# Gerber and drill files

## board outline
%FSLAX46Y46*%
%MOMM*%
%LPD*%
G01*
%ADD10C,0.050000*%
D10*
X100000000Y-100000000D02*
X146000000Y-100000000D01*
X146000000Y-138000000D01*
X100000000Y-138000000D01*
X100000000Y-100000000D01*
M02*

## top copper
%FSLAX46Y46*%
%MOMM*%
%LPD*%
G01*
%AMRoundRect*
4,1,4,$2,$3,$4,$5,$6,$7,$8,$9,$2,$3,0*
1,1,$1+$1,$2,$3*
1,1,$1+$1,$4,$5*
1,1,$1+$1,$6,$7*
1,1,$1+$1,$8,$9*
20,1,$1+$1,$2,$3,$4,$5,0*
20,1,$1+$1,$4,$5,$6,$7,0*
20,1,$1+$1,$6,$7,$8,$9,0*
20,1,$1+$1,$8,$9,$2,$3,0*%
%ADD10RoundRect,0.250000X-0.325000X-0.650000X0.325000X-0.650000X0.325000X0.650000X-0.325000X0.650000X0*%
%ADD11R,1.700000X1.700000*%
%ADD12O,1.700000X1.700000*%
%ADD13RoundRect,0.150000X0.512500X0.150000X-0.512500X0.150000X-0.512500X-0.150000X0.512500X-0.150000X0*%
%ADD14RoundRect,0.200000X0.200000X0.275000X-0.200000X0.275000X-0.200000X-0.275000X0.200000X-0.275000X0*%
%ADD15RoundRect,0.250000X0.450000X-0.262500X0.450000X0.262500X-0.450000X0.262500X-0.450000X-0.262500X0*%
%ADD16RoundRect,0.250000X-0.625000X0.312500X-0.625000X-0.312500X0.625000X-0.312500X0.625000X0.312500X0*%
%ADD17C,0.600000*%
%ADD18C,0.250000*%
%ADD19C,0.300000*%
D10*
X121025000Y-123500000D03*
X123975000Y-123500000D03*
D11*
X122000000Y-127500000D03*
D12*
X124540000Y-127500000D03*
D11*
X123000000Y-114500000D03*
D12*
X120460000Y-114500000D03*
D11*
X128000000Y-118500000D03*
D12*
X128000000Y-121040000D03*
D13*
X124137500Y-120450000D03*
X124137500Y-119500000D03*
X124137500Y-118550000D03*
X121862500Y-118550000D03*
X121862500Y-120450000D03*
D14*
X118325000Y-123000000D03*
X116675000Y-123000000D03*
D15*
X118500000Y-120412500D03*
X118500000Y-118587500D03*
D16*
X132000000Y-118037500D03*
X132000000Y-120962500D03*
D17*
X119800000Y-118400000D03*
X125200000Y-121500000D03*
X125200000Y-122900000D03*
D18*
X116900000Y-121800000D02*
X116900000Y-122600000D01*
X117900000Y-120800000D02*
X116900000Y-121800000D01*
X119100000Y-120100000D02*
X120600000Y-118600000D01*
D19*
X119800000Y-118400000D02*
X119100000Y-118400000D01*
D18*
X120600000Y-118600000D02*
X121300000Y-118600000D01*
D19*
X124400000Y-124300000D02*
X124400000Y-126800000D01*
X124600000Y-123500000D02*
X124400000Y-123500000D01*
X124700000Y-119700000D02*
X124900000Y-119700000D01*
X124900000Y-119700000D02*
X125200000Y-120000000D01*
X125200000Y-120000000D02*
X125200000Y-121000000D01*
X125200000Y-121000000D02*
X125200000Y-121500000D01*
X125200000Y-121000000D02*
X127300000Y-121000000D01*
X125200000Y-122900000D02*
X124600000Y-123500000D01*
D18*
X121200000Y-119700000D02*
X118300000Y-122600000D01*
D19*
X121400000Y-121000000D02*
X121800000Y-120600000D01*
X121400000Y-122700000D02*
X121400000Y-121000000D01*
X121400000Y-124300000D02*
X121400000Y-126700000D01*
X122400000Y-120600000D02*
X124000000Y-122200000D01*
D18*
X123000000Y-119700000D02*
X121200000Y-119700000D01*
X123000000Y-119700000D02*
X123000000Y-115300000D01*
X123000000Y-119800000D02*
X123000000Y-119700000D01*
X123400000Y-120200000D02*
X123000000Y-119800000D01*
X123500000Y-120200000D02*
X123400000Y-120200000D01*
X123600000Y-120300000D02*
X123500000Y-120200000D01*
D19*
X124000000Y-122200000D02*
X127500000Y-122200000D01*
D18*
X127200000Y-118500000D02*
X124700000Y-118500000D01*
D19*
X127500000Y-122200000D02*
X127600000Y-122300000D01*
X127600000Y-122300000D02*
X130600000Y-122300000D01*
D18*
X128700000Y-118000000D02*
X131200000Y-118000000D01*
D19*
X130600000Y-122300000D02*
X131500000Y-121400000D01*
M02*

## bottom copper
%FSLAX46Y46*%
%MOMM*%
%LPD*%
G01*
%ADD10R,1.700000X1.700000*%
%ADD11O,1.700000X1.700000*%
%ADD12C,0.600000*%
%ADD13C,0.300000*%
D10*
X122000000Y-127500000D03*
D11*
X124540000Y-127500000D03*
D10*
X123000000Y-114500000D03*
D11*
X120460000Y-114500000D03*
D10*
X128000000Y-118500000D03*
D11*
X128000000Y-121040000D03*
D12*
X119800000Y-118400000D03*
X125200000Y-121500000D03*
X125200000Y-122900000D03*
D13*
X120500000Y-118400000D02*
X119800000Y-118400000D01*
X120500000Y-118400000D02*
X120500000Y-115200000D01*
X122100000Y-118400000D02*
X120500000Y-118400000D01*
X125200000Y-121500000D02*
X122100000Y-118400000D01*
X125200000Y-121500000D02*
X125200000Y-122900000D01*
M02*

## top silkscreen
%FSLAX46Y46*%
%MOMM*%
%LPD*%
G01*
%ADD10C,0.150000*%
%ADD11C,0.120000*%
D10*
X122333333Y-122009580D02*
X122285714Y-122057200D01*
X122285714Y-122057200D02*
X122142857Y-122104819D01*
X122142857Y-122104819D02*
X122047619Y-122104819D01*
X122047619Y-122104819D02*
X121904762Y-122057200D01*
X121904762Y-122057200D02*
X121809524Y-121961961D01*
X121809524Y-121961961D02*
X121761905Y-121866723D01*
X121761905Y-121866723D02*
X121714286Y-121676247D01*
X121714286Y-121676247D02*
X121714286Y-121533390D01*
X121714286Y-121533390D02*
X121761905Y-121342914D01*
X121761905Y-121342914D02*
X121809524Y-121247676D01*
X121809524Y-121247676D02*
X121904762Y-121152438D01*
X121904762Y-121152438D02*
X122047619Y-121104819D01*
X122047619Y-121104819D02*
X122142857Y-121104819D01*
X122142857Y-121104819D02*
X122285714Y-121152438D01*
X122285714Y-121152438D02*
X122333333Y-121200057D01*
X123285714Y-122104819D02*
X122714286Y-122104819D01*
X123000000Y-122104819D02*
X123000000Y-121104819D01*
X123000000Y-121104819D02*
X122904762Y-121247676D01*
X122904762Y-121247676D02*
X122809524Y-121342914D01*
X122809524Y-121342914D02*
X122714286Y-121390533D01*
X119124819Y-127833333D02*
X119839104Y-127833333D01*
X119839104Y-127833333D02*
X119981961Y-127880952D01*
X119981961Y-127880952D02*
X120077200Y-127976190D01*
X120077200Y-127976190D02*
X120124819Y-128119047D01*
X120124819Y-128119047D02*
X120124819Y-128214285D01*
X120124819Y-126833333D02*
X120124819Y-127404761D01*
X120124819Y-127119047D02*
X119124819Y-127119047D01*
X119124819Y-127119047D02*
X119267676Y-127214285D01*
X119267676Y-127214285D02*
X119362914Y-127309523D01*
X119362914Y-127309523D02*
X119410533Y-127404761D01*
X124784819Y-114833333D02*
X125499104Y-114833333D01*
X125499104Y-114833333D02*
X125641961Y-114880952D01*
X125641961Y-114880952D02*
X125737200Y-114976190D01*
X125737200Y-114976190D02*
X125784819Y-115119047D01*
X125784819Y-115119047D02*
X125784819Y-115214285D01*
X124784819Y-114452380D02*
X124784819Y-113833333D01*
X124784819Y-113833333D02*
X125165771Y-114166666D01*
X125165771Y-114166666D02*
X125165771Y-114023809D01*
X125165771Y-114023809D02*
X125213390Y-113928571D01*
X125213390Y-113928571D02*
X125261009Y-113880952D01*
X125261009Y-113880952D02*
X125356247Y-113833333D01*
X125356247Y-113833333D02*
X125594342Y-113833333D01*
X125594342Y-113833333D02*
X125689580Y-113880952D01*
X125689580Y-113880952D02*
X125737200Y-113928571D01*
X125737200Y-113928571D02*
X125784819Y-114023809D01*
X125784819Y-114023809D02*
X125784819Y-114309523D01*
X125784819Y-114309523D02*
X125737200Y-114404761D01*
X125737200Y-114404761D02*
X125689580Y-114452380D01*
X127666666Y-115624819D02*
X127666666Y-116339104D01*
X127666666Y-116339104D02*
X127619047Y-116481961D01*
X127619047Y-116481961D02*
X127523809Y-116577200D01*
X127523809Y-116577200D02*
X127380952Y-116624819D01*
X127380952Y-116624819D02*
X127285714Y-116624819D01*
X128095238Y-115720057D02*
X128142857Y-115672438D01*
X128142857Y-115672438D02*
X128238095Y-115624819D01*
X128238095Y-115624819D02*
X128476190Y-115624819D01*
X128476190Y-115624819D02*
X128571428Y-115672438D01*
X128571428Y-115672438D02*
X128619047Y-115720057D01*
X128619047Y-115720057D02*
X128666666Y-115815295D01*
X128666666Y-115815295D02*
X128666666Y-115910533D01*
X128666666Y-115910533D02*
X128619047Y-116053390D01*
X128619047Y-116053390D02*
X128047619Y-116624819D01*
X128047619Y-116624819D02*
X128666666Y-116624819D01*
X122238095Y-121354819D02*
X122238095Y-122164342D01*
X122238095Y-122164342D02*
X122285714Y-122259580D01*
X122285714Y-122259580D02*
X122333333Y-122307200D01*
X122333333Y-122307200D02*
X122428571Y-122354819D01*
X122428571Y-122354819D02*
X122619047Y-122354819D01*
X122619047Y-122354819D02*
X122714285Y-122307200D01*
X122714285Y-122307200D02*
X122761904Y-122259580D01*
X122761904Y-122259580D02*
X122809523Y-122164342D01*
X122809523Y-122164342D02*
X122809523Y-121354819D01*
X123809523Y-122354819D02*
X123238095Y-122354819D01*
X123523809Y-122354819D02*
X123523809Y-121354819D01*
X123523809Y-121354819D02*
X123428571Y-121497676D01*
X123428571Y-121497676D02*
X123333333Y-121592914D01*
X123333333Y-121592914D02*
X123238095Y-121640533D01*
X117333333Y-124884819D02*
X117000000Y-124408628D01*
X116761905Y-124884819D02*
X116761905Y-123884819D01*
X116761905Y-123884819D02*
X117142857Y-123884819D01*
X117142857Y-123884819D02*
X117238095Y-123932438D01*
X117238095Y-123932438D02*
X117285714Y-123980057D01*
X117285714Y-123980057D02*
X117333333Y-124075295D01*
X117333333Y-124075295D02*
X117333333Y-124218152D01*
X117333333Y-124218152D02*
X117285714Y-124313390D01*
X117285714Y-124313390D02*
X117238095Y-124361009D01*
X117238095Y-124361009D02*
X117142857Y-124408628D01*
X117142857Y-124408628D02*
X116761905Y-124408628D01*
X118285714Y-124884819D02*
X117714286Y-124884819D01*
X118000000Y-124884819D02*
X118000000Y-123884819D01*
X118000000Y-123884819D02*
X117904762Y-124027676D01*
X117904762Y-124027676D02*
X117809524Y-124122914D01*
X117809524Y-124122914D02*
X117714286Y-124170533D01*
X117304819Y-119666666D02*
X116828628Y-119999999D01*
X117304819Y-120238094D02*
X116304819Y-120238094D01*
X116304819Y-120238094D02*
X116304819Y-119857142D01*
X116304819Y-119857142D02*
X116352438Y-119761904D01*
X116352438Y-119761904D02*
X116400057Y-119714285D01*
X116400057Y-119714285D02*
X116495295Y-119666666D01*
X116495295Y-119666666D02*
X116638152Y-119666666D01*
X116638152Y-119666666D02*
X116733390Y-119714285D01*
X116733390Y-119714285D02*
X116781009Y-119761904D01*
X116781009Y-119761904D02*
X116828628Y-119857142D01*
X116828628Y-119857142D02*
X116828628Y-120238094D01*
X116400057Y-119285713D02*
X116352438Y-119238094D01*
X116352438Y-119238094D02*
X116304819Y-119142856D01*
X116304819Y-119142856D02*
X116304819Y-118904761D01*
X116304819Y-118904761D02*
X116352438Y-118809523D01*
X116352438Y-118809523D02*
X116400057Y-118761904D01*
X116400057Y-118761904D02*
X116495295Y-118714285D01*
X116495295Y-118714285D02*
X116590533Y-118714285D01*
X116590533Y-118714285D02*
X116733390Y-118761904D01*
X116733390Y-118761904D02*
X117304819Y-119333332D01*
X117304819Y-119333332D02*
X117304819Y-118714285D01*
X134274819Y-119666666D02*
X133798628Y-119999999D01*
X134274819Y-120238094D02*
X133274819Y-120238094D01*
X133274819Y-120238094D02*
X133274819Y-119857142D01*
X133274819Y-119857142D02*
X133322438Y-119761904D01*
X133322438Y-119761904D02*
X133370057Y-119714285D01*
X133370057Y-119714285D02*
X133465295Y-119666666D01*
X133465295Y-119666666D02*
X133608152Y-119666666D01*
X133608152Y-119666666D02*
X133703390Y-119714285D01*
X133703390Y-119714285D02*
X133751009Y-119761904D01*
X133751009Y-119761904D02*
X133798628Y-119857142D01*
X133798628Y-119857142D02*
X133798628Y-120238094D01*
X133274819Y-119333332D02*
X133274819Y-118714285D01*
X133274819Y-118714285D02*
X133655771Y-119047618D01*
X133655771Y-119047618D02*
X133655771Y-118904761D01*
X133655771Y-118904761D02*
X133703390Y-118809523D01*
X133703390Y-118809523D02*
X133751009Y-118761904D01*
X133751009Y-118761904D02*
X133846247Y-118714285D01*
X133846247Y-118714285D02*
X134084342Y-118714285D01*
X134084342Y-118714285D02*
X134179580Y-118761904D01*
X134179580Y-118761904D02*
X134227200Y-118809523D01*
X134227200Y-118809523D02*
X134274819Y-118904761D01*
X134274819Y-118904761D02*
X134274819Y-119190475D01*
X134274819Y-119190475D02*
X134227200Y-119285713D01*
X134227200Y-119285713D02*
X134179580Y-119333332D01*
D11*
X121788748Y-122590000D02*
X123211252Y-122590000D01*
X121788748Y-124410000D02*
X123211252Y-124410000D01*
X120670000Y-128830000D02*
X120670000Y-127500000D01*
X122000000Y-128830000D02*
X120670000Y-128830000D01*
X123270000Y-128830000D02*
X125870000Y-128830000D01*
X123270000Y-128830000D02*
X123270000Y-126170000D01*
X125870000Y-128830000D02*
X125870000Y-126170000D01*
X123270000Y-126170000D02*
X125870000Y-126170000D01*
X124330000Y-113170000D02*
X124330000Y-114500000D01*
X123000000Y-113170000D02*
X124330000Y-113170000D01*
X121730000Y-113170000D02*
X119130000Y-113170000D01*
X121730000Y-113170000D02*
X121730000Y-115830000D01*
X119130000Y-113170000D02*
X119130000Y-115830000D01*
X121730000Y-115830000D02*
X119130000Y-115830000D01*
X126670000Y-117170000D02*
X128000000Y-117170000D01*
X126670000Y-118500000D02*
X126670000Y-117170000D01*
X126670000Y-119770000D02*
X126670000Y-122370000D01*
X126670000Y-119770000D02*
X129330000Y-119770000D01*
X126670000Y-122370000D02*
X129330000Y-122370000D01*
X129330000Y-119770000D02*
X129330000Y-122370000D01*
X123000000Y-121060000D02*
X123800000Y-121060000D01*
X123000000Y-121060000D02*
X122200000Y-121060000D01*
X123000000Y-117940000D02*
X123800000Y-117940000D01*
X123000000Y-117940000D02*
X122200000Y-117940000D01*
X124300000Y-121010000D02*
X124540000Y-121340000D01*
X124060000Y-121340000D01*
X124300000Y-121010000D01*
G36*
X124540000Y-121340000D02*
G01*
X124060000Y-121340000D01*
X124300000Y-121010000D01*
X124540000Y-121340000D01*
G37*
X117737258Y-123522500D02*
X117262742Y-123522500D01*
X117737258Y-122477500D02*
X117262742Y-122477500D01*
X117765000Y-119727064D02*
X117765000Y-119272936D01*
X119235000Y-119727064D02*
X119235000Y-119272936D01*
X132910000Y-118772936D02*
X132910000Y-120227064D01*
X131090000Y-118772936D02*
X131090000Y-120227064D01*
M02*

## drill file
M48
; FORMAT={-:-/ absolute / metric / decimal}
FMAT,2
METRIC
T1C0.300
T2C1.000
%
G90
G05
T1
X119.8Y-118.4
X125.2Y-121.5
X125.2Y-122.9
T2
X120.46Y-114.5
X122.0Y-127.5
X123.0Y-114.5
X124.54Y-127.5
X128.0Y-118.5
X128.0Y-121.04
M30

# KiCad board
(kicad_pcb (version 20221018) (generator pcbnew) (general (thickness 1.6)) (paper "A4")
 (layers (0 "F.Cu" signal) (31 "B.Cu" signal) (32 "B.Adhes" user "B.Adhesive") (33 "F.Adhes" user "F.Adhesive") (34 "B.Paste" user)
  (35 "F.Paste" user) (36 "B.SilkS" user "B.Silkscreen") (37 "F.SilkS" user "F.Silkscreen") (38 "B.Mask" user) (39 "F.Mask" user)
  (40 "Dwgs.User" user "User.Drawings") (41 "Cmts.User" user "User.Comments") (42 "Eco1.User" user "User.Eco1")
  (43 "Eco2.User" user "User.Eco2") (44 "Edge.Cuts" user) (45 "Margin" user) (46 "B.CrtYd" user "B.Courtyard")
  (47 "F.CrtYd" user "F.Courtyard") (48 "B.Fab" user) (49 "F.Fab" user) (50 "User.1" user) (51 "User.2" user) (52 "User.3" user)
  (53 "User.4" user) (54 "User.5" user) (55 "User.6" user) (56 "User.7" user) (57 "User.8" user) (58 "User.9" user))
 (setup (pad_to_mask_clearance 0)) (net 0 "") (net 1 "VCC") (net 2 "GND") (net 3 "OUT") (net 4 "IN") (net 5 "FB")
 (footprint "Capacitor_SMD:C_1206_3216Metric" (layer "F.Cu") (at 122.5 123.5)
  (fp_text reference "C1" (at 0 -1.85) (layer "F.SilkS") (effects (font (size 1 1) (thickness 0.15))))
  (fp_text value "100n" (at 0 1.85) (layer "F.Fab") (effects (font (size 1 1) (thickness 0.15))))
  (fp_line (start -0.711252 -0.91) (end 0.711252 -0.91) (stroke (width 0.12) (type solid)) (layer "F.SilkS"))
  (fp_line (start -0.711252 0.91) (end 0.711252 0.91) (stroke (width 0.12) (type solid)) (layer "F.SilkS"))
  (pad "1" smd roundrect (at -1.475 0) (size 1.15 1.8) (layers "F.Cu" "F.Paste" "F.Mask") (roundrect_rratio 0.217391) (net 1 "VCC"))
  (pad "2" smd roundrect (at 1.475 0) (size 1.15 1.8) (layers "F.Cu" "F.Paste" "F.Mask") (roundrect_rratio 0.217391) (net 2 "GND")))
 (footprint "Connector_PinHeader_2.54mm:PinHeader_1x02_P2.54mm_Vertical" (layer "F.Cu") (at 122 127.5 90)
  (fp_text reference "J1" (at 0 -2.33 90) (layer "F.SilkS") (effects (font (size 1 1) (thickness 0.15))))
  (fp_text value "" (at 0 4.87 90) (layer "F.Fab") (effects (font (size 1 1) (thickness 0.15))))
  (fp_line (start -1.33 -1.33) (end 0 -1.33) (stroke (width 0.12) (type solid)) (layer "F.SilkS"))
  (fp_line (start -1.33 0) (end -1.33 -1.33) (stroke (width 0.12) (type solid)) (layer "F.SilkS"))
  (fp_line (start -1.33 1.27) (end -1.33 3.87) (stroke (width 0.12) (type solid)) (layer "F.SilkS"))
  (fp_line (start -1.33 1.27) (end 1.33 1.27) (stroke (width 0.12) (type solid)) (layer "F.SilkS"))
  (fp_line (start -1.33 3.87) (end 1.33 3.87) (stroke (width 0.12) (type solid)) (layer "F.SilkS"))
  (fp_line (start 1.33 1.27) (end 1.33 3.87) (stroke (width 0.12) (type solid)) (layer "F.SilkS"))
  (pad "1" thru_hole rect (at 0 0 90) (size 1.7 1.7) (drill 1) (layers "*.Cu" "*.Mask") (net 1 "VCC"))
  (pad "2" thru_hole oval (at 0 2.54 90) (size 1.7 1.7) (drill 1) (layers "*.Cu" "*.Mask") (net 2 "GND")))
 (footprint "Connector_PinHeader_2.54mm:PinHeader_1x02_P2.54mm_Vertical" (layer "F.Cu") (at 123 114.5 -90)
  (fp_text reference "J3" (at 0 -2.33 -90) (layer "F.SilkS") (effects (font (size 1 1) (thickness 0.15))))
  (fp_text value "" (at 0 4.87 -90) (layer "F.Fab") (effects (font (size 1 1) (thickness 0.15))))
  (fp_line (start -1.33 -1.33) (end 0 -1.33) (stroke (width 0.12) (type solid)) (layer "F.SilkS"))
  (fp_line (start -1.33 0) (end -1.33 -1.33) (stroke (width 0.12) (type solid)) (layer "F.SilkS"))
  (fp_line (start -1.33 1.27) (end -1.33 3.87) (stroke (width 0.12) (type solid)) (layer "F.SilkS"))
  (fp_line (start -1.33 1.27) (end 1.33 1.27) (stroke (width 0.12) (type solid)) (layer "F.SilkS"))
  (fp_line (start -1.33 3.87) (end 1.33 3.87) (stroke (width 0.12) (type solid)) (layer "F.SilkS"))
  (fp_line (start 1.33 1.27) (end 1.33 3.87) (stroke (width 0.12) (type solid)) (layer "F.SilkS"))
  (pad "1" thru_hole rect (at 0 0 270) (size 1.7 1.7) (drill 1) (layers "*.Cu" "*.Mask") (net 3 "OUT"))
  (pad "2" thru_hole oval (at 0 2.54 270) (size 1.7 1.7) (drill 1) (layers "*.Cu" "*.Mask") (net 2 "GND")))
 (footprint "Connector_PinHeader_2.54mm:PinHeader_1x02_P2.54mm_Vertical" (layer "F.Cu") (at 128 118.5)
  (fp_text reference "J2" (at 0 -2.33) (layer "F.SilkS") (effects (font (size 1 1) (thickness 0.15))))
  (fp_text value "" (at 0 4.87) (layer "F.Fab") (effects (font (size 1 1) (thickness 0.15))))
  (fp_line (start -1.33 -1.33) (end 0 -1.33) (stroke (width 0.12) (type solid)) (layer "F.SilkS"))
  (fp_line (start -1.33 0) (end -1.33 -1.33) (stroke (width 0.12) (type solid)) (layer "F.SilkS"))
  (fp_line (start -1.33 1.27) (end -1.33 3.87) (stroke (width 0.12) (type solid)) (layer "F.SilkS"))
  (fp_line (start -1.33 1.27) (end 1.33 1.27) (stroke (width 0.12) (type solid)) (layer "F.SilkS"))
  (fp_line (start -1.33 3.87) (end 1.33 3.87) (stroke (width 0.12) (type solid)) (layer "F.SilkS"))
  (fp_line (start 1.33 1.27) (end 1.33 3.87) (stroke (width 0.12) (type solid)) (layer "F.SilkS"))
  (pad "1" thru_hole rect (at 0 0) (size 1.7 1.7) (drill 1) (layers "*.Cu" "*.Mask") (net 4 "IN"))
  (pad "2" thru_hole oval (at 0 2.54) (size 1.7 1.7) (drill 1) (layers "*.Cu" "*.Mask") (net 2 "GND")))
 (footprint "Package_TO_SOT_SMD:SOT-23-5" (layer "F.Cu") (at 123 119.5 180)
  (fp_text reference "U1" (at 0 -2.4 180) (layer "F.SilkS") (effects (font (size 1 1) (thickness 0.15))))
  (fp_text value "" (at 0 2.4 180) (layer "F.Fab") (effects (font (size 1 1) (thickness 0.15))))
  (fp_line (start 0 -1.56) (end -0.8 -1.56) (stroke (width 0.12) (type solid)) (layer "F.SilkS"))
  (fp_line (start 0 -1.56) (end 0.8 -1.56) (stroke (width 0.12) (type solid)) (layer "F.SilkS"))
  (fp_line (start 0 1.56) (end -0.8 1.56) (stroke (width 0.12) (type solid)) (layer "F.SilkS"))
  (fp_line (start 0 1.56) (end 0.8 1.56) (stroke (width 0.12) (type solid)) (layer "F.SilkS"))
  (fp_poly
   (pts (xy -1.3 -1.51) (xy -1.54 -1.84) (xy -1.06 -1.84) (xy -1.3 -1.51)) (stroke (width 0.12) (type solid)) (fill solid) (layer "F.SilkS"))
  (pad "1" smd roundrect (at -1.1375 -0.95 180) (size 1.325 0.6) (layers "F.Cu" "F.Paste" "F.Mask") (roundrect_rratio 0.25) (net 3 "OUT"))
  (pad "2" smd roundrect (at -1.1375 0 180) (size 1.325 0.6) (layers "F.Cu" "F.Paste" "F.Mask") (roundrect_rratio 0.25) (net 2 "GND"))
  (pad "3" smd roundrect (at -1.1375 0.95 180) (size 1.325 0.6) (layers "F.Cu" "F.Paste" "F.Mask") (roundrect_rratio 0.25) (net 4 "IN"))
  (pad "4" smd roundrect (at 1.1375 0.95 180) (size 1.325 0.6) (layers "F.Cu" "F.Paste" "F.Mask") (roundrect_rratio 0.25) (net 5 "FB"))
  (pad "5" smd roundrect (at 1.1375 -0.95 180) (size 1.325 0.6) (layers "F.Cu" "F.Paste" "F.Mask") (roundrect_rratio 0.25) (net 1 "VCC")))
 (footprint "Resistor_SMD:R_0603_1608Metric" (layer "F.Cu") (at 117.5 123 180)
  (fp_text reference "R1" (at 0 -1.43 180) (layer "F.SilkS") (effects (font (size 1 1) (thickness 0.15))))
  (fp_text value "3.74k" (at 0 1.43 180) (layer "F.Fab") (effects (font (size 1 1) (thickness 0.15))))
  (fp_line (start -0.237258 -0.5225) (end 0.237258 -0.5225) (stroke (width 0.12) (type solid)) (layer "F.SilkS"))
  (fp_line (start -0.237258 0.5225) (end 0.237258 0.5225) (stroke (width 0.12) (type solid)) (layer "F.SilkS"))
  (pad "1" smd roundrect (at -0.825 0 180) (size 0.8 0.95) (layers "F.Cu" "F.Paste" "F.Mask") (roundrect_rratio 0.25) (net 3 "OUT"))
  (pad "2" smd roundrect (at 0.825 0 180) (size 0.8 0.95) (layers "F.Cu" "F.Paste" "F.Mask") (roundrect_rratio 0.25) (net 5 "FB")))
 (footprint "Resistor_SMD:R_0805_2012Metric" (layer "F.Cu") (at 118.5 119.5 90)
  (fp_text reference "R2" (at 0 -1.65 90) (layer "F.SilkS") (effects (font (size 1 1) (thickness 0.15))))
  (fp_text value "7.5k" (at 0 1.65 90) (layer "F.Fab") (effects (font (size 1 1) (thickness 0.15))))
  (fp_line (start -0.227064 -0.735) (end 0.227064 -0.735) (stroke (width 0.12) (type solid)) (layer "F.SilkS"))
  (fp_line (start -0.227064 0.735) (end 0.227064 0.735) (stroke (width 0.12) (type solid)) (layer "F.SilkS"))
  (pad "1" smd roundrect (at -0.9125 0 90) (size 1.025 1.4) (layers "F.Cu" "F.Paste" "F.Mask") (roundrect_rratio 0.243902) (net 5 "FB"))
  (pad "2" smd roundrect (at 0.9125 0 90) (size 1.025 1.4) (layers "F.Cu" "F.Paste" "F.Mask") (roundrect_rratio 0.243902) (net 2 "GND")))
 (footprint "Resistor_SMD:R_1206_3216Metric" (layer "F.Cu") (at 132 119.5 -90)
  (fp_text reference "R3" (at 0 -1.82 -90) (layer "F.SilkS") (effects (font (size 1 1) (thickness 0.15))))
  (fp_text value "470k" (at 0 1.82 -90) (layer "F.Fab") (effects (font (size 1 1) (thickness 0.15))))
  (fp_line (start -0.727064 -0.91) (end 0.727064 -0.91) (stroke (width 0.12) (type solid)) (layer "F.SilkS"))
  (fp_line (start -0.727064 0.91) (end 0.727064 0.91) (stroke (width 0.12) (type solid)) (layer "F.SilkS"))
  (pad "1" smd roundrect (at -1.4625 0 270) (size 1.125 1.75) (layers "F.Cu" "F.Paste" "F.Mask") (roundrect_rratio 0.222222) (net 4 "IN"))
  (pad "2" smd roundrect (at 1.4625 0 270) (size 1.125 1.75) (layers "F.Cu" "F.Paste" "F.Mask") (roundrect_rratio 0.222222) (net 1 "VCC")))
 (gr_rect (start 100 100) (end 146 138) (stroke (width 0.05) (type default)) (fill none) (layer "Edge.Cuts"))
 (segment (start 116.9 121.8) (end 116.9 122.6) (width 0.25) (layer "F.Cu") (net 5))
 (segment (start 117.9 120.8) (end 116.9 121.8) (width 0.25) (layer "F.Cu") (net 5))
 (segment (start 119.1 120.1) (end 120.6 118.6) (width 0.25) (layer "F.Cu") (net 5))
 (segment (start 119.8 118.4) (end 119.1 118.4) (width 0.3) (layer "F.Cu") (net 2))
 (segment (start 120.6 118.6) (end 121.3 118.6) (width 0.25) (layer "F.Cu") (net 5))
 (segment (start 124.4 124.3) (end 124.4 126.8) (width 0.3) (layer "F.Cu") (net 2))
 (segment (start 124.6 123.5) (end 124.4 123.5) (width 0.3) (layer "F.Cu") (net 2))
 (segment (start 124.7 119.7) (end 124.9 119.7) (width 0.3) (layer "F.Cu") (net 2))
 (segment (start 124.9 119.7) (end 125.2 120) (width 0.3) (layer "F.Cu") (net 2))
 (segment (start 125.2 120) (end 125.2 121) (width 0.3) (layer "F.Cu") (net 2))
 (segment (start 125.2 121) (end 125.2 121.5) (width 0.3) (layer "F.Cu") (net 2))
 (segment (start 125.2 121) (end 127.3 121) (width 0.3) (layer "F.Cu") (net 2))
 (segment (start 125.2 122.9) (end 124.6 123.5) (width 0.3) (layer "F.Cu") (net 2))
 (via (at 119.8 118.4) (size 0.6) (drill 0.3) (layers "F.Cu" "B.Cu") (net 2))
 (via (at 125.2 121.5) (size 0.6) (drill 0.3) (layers "F.Cu" "B.Cu") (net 2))
 (via (at 125.2 122.9) (size 0.6) (drill 0.3) (layers "F.Cu" "B.Cu") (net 2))
 (segment (start 120.5 118.4) (end 119.8 118.4) (width 0.3) (layer "B.Cu") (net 2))
 (segment (start 120.5 118.4) (end 120.5 115.2) (width 0.3) (layer "B.Cu") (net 2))
 (segment (start 121.2 119.7) (end 118.3 122.6) (width 0.25) (layer "F.Cu") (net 3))
 (segment (start 121.4 121) (end 121.8 120.6) (width 0.3) (layer "F.Cu") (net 1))
 (segment (start 121.4 122.7) (end 121.4 121) (width 0.3) (layer "F.Cu") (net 1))
 (segment (start 121.4 124.3) (end 121.4 126.7) (width 0.3) (layer "F.Cu") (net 1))
 (segment (start 122.1 118.4) (end 120.5 118.4) (width 0.3) (layer "B.Cu") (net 2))
 (segment (start 122.4 120.6) (end 124 122.2) (width 0.3) (layer "F.Cu") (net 1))
 (segment (start 123 119.7) (end 121.2 119.7) (width 0.25) (layer "F.Cu") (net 3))
 (segment (start 123 119.7) (end 123 115.3) (width 0.25) (layer "F.Cu") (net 3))
 (segment (start 123 119.8) (end 123 119.7) (width 0.25) (layer "F.Cu") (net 3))
 (segment (start 123.4 120.2) (end 123 119.8) (width 0.25) (layer "F.Cu") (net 3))
 (segment (start 123.5 120.2) (end 123.4 120.2) (width 0.25) (layer "F.Cu") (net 3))
 (segment (start 123.6 120.3) (end 123.5 120.2) (width 0.25) (layer "F.Cu") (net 3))
 (segment (start 124 122.2) (end 127.5 122.2) (width 0.3) (layer "F.Cu") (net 1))
 (segment (start 125.2 121.5) (end 122.1 118.4) (width 0.3) (layer "B.Cu") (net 2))
 (segment (start 125.2 121.5) (end 125.2 122.9) (width 0.3) (layer "B.Cu") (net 2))
 (segment (start 127.2 118.5) (end 124.7 118.5) (width 0.25) (layer "F.Cu") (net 4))
 (segment (start 127.5 122.2) (end 127.6 122.3) (width 0.3) (layer "F.Cu") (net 1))
 (segment (start 127.6 122.3) (end 130.6 122.3) (width 0.3) (layer "F.Cu") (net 1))
 (segment (start 128.7 118) (end 131.2 118) (width 0.25) (layer "F.Cu") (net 4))
 (segment (start 130.6 122.3) (end 131.5 121.4) (width 0.3) (layer "F.Cu") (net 1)))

